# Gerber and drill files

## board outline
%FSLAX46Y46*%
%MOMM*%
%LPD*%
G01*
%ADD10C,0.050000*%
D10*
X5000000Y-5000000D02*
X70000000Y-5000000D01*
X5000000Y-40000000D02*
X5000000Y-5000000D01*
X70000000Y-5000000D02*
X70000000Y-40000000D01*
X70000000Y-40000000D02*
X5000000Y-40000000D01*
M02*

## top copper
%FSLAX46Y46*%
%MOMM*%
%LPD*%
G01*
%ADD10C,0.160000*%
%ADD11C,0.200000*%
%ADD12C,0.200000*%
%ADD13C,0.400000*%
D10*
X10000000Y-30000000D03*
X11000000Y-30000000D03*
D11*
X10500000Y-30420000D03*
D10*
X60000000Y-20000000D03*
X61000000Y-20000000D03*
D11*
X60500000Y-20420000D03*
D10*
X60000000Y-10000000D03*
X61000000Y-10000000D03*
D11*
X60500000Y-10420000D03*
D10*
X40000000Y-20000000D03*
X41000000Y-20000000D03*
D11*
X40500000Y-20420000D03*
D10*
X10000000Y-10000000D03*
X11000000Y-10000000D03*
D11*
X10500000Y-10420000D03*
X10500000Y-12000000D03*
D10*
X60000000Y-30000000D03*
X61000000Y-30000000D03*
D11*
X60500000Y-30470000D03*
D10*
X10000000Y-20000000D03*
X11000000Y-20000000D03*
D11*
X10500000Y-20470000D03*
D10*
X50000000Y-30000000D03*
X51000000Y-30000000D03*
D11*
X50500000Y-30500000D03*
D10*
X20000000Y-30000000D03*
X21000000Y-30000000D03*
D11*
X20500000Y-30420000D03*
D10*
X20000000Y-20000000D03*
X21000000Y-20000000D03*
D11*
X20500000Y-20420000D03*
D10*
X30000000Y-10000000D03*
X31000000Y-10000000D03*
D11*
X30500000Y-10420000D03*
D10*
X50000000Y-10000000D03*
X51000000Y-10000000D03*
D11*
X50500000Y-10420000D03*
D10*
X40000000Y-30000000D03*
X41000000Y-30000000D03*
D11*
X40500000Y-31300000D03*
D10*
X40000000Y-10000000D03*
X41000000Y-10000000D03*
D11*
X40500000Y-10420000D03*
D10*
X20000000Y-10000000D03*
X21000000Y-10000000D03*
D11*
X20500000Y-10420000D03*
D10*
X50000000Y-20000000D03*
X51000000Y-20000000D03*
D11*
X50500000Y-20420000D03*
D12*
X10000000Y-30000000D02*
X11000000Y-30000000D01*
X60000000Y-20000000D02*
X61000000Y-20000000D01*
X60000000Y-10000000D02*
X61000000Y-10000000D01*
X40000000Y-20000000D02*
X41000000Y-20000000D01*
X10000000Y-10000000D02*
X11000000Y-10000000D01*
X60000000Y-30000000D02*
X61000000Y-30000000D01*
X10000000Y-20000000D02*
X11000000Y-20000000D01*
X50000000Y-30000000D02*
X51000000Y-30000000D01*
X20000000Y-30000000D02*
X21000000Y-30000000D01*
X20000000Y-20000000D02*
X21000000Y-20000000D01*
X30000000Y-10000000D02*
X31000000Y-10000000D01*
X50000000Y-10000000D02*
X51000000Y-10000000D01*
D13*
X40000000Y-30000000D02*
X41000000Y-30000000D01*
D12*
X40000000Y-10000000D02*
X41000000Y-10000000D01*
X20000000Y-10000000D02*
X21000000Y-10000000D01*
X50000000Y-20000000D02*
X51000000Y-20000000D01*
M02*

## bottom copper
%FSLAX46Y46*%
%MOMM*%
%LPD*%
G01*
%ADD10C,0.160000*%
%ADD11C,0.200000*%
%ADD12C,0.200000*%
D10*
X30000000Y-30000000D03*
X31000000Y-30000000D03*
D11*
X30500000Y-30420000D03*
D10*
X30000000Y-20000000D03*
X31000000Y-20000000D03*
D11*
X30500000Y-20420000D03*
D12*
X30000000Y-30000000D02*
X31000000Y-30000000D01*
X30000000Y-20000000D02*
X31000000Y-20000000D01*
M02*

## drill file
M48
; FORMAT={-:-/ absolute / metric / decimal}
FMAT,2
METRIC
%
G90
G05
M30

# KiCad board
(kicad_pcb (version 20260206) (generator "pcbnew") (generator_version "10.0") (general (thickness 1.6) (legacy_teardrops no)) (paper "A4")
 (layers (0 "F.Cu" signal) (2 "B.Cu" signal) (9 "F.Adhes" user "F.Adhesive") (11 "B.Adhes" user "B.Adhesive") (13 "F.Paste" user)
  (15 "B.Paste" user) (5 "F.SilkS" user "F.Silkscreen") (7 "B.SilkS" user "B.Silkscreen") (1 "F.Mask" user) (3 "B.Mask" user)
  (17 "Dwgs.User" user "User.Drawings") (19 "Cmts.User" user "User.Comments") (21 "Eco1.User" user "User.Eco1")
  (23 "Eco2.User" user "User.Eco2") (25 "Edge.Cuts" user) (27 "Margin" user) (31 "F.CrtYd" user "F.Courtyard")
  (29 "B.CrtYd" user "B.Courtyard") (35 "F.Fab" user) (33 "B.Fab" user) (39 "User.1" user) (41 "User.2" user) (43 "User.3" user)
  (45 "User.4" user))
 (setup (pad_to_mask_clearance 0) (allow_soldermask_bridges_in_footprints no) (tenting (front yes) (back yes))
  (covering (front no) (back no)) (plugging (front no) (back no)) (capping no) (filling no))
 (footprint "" (layer "F.Cu") (at 10 30)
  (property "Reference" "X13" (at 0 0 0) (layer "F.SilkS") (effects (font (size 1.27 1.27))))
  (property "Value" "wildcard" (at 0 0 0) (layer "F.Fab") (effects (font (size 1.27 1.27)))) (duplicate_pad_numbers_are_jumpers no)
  (pad "1" smd circle (at 0 0) (size 0.16 0.16) (layers "F.Cu") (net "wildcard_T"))
  (pad "2" smd circle (at 1 0) (size 0.16 0.16) (layers "F.Cu") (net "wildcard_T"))
  (pad "3" smd circle (at 0.5 0.42) (size 0.2 0.2) (layers "F.Cu") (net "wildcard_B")))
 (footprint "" (layer "F.Cu") (at 60 20)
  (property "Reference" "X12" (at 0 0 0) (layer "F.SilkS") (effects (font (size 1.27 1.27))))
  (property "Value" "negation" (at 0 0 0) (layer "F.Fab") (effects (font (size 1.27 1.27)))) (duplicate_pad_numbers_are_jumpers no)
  (pad "1" smd circle (at 0 0) (size 0.16 0.16) (layers "F.Cu") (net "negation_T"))
  (pad "2" smd circle (at 1 0) (size 0.16 0.16) (layers "F.Cu") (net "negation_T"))
  (pad "3" smd circle (at 0.5 0.42) (size 0.2 0.2) (layers "F.Cu") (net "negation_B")))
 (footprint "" (layer "F.Cu") (at 60 10)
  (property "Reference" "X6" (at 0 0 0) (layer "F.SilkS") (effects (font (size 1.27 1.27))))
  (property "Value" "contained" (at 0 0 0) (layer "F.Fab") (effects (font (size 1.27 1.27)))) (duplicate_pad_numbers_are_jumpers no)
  (pad "1" smd circle (at 0 0) (size 0.16 0.16) (layers "F.Cu") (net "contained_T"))
  (pad "2" smd circle (at 1 0) (size 0.16 0.16) (layers "F.Cu") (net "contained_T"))
  (pad "3" smd circle (at 0.5 0.42) (size 0.2 0.2) (layers "F.Cu") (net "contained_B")))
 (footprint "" (layer "F.Cu") (at 40 20)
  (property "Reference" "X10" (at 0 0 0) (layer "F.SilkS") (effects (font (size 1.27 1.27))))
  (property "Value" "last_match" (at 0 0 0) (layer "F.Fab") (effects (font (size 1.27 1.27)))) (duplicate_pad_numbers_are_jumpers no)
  (pad "1" smd circle (at 0 0) (size 0.16 0.16) (layers "F.Cu") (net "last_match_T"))
  (pad "2" smd circle (at 1 0) (size 0.16 0.16) (layers "F.Cu") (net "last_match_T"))
  (pad "3" smd circle (at 0.5 0.42) (size 0.2 0.2) (layers "F.Cu") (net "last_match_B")))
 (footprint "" (layer "F.Cu") (at 10 10)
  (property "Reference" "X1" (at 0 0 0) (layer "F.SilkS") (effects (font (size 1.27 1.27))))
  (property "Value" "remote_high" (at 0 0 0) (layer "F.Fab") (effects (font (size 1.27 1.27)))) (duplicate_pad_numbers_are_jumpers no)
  (pad "1" smd circle (at 0 0) (size 0.16 0.16) (layers "F.Cu") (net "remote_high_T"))
  (pad "2" smd circle (at 1 0) (size 0.16 0.16) (layers "F.Cu") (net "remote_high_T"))
  (pad "3" smd circle (at 0.5 0.42) (size 0.2 0.2) (layers "F.Cu") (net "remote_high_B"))
  (pad "4" smd circle (at 0.5 2) (size 0.2 0.2) (layers "F.Cu") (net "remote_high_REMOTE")))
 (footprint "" (layer "F.Cu") (at 60 30)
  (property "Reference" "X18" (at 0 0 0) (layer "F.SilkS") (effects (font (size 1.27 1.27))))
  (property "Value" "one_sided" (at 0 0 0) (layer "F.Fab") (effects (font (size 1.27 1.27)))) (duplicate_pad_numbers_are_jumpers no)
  (pad "1" smd circle (at 0 0) (size 0.16 0.16) (layers "F.Cu") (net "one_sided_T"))
  (pad "2" smd circle (at 1 0) (size 0.16 0.16) (layers "F.Cu") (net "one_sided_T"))
  (pad "3" smd circle (at 0.5 0.47) (size 0.2 0.2) (layers "F.Cu") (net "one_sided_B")))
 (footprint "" (layer "F.Cu") (at 10 20)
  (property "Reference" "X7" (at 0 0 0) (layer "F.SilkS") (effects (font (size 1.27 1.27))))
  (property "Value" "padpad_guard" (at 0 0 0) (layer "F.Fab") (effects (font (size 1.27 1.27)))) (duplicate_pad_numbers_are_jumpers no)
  (pad "1" smd circle (at 0 0) (size 0.16 0.16) (layers "F.Cu") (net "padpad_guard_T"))
  (pad "2" smd circle (at 1 0) (size 0.16 0.16) (layers "F.Cu") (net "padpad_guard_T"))
  (pad "3" smd circle (at 0.5 0.47) (size 0.2 0.2) (layers "F.Cu") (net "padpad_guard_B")))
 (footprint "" (layer "F.Cu") (at 50 30)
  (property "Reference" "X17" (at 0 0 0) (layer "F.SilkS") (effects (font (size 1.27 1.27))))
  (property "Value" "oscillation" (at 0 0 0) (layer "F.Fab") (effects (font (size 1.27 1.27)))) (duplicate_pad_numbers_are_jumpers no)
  (pad "1" smd circle (at 0 0) (size 0.16 0.16) (layers "F.Cu") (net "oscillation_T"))
  (pad "2" smd circle (at 1 0) (size 0.16 0.16) (layers "F.Cu") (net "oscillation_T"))
  (pad "3" smd circle (at 0.5 0.5) (size 0.2 0.2) (layers "F.Cu") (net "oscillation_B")))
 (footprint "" (layer "F.Cu") (at 20 30)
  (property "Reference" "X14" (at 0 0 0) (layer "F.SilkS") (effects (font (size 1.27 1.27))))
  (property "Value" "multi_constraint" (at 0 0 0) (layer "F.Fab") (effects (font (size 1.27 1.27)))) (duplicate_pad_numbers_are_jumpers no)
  (pad "1" smd circle (at 0 0) (size 0.16 0.16) (layers "F.Cu") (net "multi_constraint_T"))
  (pad "2" smd circle (at 1 0) (size 0.16 0.16) (layers "F.Cu") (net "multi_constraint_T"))
  (pad "3" smd circle (at 0.5 0.42) (size 0.2 0.2) (layers "F.Cu") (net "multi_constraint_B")))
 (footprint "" (layer "F.Cu") (at 30 30)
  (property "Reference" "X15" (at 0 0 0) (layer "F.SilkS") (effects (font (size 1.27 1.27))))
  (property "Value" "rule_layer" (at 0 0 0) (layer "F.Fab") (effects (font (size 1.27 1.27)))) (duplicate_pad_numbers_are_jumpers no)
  (pad "1" smd circle (at 0 0) (size 0.16 0.16) (layers "B.Cu") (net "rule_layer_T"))
  (pad "2" smd circle (at 1 0) (size 0.16 0.16) (layers "B.Cu") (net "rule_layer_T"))
  (pad "3" smd circle (at 0.5 0.42) (size 0.2 0.2) (layers "B.Cu") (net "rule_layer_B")))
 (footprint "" (layer "F.Cu") (at 20 20)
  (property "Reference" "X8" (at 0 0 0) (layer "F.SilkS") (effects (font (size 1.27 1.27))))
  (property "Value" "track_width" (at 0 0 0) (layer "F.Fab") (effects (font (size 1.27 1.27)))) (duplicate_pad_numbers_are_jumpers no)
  (pad "1" smd circle (at 0 0) (size 0.16 0.16) (layers "F.Cu") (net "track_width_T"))
  (pad "2" smd circle (at 1 0) (size 0.16 0.16) (layers "F.Cu") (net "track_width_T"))
  (pad "3" smd circle (at 0.5 0.42) (size 0.2 0.2) (layers "F.Cu") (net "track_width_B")))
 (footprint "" (layer "F.Cu") (at 30 10)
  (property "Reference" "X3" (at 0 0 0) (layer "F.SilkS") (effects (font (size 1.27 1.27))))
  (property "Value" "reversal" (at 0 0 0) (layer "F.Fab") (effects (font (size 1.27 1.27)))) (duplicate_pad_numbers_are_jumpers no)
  (pad "1" smd circle (at 0 0) (size 0.16 0.16) (layers "F.Cu") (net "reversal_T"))
  (pad "2" smd circle (at 1 0) (size 0.16 0.16) (layers "F.Cu") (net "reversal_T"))
  (pad "3" smd circle (at 0.5 0.42) (size 0.2 0.2) (layers "F.Cu") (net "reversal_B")))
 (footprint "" (layer "F.Cu") (at 50 10)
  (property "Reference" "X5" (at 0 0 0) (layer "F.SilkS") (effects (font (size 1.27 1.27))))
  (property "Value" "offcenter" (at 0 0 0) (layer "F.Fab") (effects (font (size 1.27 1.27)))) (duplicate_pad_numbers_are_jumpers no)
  (pad "1" smd circle (at 0 0) (size 0.16 0.16) (layers "F.Cu") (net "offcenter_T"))
  (pad "2" smd circle (at 1 0) (size 0.16 0.16) (layers "F.Cu") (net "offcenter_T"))
  (pad "3" smd circle (at 0.5 0.42) (size 0.2 0.2) (layers "F.Cu") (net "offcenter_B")))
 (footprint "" (layer "F.Cu") (at 40 30)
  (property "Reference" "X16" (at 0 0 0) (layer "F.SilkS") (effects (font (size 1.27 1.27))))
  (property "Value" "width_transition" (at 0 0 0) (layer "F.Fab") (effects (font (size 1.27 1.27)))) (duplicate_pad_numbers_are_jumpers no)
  (pad "1" smd circle (at 0 0) (size 0.16 0.16) (layers "F.Cu") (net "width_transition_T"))
  (pad "2" smd circle (at 1 0) (size 0.16 0.16) (layers "F.Cu") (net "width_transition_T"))
  (pad "3" smd circle (at 0.5 1.3) (size 0.2 0.2) (layers "F.Cu") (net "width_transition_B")))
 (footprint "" (layer "F.Cu") (at 30 20)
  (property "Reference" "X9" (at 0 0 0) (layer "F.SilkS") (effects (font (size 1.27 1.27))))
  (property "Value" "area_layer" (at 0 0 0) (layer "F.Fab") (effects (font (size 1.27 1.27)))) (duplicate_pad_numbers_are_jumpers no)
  (pad "1" smd circle (at 0 0) (size 0.16 0.16) (layers "B.Cu") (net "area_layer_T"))
  (pad "2" smd circle (at 1 0) (size 0.16 0.16) (layers "B.Cu") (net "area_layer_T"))
  (pad "3" smd circle (at 0.5 0.42) (size 0.2 0.2) (layers "B.Cu") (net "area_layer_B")))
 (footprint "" (layer "F.Cu") (at 40 10)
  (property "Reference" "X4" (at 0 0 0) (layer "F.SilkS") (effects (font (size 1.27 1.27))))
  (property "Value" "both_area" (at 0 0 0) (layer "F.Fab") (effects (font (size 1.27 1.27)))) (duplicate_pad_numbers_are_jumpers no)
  (pad "1" smd circle (at 0 0) (size 0.16 0.16) (layers "F.Cu") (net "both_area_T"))
  (pad "2" smd circle (at 1 0) (size 0.16 0.16) (layers "F.Cu") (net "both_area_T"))
  (pad "3" smd circle (at 0.5 0.42) (size 0.2 0.2) (layers "F.Cu") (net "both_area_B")))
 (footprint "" (layer "F.Cu") (at 20 10)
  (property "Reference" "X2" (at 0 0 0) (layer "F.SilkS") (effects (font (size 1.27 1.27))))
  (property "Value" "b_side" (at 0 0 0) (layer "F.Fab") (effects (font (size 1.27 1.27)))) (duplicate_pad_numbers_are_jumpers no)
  (pad "1" smd circle (at 0 0) (size 0.16 0.16) (layers "F.Cu") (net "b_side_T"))
  (pad "2" smd circle (at 1 0) (size 0.16 0.16) (layers "F.Cu") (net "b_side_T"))
  (pad "3" smd circle (at 0.5 0.42) (size 0.2 0.2) (layers "F.Cu") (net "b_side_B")))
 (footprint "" (layer "F.Cu") (at 50 20)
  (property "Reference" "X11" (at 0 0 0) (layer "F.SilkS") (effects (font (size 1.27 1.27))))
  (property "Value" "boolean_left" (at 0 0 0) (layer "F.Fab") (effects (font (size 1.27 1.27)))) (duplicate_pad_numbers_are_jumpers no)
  (pad "1" smd circle (at 0 0) (size 0.16 0.16) (layers "F.Cu") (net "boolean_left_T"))
  (pad "2" smd circle (at 1 0) (size 0.16 0.16) (layers "F.Cu") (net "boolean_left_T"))
  (pad "3" smd circle (at 0.5 0.42) (size 0.2 0.2) (layers "F.Cu") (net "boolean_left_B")))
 (gr_line (start 5 5) (end 70 5) (stroke (width 0.05) (type default)) (layer "Edge.Cuts"))
 (gr_line (start 5 40) (end 5 5) (stroke (width 0.05) (type default)) (layer "Edge.Cuts"))
 (gr_line (start 70 5) (end 70 40) (stroke (width 0.05) (type default)) (layer "Edge.Cuts"))
 (gr_line (start 70 40) (end 5 40) (stroke (width 0.05) (type default)) (layer "Edge.Cuts"))
 (segment (start 10 30) (end 11 30) (width 0.2) (layer "F.Cu") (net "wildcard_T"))
 (segment (start 60 20) (end 61 20) (width 0.2) (layer "F.Cu") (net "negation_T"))
 (segment (start 60 10) (end 61 10) (width 0.2) (layer "F.Cu") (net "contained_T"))
 (segment (start 40 20) (end 41 20) (width 0.2) (layer "F.Cu") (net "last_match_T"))
 (segment (start 10 10) (end 11 10) (width 0.2) (layer "F.Cu") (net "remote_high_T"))
 (segment (start 60 30) (end 61 30) (width 0.2) (layer "F.Cu") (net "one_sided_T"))
 (segment (start 10 20) (end 11 20) (width 0.2) (layer "F.Cu") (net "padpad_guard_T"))
 (segment (start 50 30) (end 51 30) (width 0.2) (layer "F.Cu") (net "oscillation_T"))
 (segment (start 20 30) (end 21 30) (width 0.2) (layer "F.Cu") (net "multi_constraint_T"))
 (segment (start 30 30) (end 31 30) (width 0.2) (layer "B.Cu") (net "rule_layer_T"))
 (segment (start 20 20) (end 21 20) (width 0.2) (layer "F.Cu") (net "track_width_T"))
 (segment (start 30 10) (end 31 10) (width 0.2) (layer "F.Cu") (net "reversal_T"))
 (segment (start 50 10) (end 51 10) (width 0.2) (layer "F.Cu") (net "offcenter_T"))
 (segment (start 40 30) (end 41 30) (width 0.4) (layer "F.Cu") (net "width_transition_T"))
 (segment (start 30 20) (end 31 20) (width 0.2) (layer "B.Cu") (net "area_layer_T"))
 (segment (start 40 10) (end 41 10) (width 0.2) (layer "F.Cu") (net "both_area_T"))
 (segment (start 20 10) (end 21 10) (width 0.2) (layer "F.Cu") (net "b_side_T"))
 (segment (start 50 20) (end 51 20) (width 0.2) (layer "F.Cu") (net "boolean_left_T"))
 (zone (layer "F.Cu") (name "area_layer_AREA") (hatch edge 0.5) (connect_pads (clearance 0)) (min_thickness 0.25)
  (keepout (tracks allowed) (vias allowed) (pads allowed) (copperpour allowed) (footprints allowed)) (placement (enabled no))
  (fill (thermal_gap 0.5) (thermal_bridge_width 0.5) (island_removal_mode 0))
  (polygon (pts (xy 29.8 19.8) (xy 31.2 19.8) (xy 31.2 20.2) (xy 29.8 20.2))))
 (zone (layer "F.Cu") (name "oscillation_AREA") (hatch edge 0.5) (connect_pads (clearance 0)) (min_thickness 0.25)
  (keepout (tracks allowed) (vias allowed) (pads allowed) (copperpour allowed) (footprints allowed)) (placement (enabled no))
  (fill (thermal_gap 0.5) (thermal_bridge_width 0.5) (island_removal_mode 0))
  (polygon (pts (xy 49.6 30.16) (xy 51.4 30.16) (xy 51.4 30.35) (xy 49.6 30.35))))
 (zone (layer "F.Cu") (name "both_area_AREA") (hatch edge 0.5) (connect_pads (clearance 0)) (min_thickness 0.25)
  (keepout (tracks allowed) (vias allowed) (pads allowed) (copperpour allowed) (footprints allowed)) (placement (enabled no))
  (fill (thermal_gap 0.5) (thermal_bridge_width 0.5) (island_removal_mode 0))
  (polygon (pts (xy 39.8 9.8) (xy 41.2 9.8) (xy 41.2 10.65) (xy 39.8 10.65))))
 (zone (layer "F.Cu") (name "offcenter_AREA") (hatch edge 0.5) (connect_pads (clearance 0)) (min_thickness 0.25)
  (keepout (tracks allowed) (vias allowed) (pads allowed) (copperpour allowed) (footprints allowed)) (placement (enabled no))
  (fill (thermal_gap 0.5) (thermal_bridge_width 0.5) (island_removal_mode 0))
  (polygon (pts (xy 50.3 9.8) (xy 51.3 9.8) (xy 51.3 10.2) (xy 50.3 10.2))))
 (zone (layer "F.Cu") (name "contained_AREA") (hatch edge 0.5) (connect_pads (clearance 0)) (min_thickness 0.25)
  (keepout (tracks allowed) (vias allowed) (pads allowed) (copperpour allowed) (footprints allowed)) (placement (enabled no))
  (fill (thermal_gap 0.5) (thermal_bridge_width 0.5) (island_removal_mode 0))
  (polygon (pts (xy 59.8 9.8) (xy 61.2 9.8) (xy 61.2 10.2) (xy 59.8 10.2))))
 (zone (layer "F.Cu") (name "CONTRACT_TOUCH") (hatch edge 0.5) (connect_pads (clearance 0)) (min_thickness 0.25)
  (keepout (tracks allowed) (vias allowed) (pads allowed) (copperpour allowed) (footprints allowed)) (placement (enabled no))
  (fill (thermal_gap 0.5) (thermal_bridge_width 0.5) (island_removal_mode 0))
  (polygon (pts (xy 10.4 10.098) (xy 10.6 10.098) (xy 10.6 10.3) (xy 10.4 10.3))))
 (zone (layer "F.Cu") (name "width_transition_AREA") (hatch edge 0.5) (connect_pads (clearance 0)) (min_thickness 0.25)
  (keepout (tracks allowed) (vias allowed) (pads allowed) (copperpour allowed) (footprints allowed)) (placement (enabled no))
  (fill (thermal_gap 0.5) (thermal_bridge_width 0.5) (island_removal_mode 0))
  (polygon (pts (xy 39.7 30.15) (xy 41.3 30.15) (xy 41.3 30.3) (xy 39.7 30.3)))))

